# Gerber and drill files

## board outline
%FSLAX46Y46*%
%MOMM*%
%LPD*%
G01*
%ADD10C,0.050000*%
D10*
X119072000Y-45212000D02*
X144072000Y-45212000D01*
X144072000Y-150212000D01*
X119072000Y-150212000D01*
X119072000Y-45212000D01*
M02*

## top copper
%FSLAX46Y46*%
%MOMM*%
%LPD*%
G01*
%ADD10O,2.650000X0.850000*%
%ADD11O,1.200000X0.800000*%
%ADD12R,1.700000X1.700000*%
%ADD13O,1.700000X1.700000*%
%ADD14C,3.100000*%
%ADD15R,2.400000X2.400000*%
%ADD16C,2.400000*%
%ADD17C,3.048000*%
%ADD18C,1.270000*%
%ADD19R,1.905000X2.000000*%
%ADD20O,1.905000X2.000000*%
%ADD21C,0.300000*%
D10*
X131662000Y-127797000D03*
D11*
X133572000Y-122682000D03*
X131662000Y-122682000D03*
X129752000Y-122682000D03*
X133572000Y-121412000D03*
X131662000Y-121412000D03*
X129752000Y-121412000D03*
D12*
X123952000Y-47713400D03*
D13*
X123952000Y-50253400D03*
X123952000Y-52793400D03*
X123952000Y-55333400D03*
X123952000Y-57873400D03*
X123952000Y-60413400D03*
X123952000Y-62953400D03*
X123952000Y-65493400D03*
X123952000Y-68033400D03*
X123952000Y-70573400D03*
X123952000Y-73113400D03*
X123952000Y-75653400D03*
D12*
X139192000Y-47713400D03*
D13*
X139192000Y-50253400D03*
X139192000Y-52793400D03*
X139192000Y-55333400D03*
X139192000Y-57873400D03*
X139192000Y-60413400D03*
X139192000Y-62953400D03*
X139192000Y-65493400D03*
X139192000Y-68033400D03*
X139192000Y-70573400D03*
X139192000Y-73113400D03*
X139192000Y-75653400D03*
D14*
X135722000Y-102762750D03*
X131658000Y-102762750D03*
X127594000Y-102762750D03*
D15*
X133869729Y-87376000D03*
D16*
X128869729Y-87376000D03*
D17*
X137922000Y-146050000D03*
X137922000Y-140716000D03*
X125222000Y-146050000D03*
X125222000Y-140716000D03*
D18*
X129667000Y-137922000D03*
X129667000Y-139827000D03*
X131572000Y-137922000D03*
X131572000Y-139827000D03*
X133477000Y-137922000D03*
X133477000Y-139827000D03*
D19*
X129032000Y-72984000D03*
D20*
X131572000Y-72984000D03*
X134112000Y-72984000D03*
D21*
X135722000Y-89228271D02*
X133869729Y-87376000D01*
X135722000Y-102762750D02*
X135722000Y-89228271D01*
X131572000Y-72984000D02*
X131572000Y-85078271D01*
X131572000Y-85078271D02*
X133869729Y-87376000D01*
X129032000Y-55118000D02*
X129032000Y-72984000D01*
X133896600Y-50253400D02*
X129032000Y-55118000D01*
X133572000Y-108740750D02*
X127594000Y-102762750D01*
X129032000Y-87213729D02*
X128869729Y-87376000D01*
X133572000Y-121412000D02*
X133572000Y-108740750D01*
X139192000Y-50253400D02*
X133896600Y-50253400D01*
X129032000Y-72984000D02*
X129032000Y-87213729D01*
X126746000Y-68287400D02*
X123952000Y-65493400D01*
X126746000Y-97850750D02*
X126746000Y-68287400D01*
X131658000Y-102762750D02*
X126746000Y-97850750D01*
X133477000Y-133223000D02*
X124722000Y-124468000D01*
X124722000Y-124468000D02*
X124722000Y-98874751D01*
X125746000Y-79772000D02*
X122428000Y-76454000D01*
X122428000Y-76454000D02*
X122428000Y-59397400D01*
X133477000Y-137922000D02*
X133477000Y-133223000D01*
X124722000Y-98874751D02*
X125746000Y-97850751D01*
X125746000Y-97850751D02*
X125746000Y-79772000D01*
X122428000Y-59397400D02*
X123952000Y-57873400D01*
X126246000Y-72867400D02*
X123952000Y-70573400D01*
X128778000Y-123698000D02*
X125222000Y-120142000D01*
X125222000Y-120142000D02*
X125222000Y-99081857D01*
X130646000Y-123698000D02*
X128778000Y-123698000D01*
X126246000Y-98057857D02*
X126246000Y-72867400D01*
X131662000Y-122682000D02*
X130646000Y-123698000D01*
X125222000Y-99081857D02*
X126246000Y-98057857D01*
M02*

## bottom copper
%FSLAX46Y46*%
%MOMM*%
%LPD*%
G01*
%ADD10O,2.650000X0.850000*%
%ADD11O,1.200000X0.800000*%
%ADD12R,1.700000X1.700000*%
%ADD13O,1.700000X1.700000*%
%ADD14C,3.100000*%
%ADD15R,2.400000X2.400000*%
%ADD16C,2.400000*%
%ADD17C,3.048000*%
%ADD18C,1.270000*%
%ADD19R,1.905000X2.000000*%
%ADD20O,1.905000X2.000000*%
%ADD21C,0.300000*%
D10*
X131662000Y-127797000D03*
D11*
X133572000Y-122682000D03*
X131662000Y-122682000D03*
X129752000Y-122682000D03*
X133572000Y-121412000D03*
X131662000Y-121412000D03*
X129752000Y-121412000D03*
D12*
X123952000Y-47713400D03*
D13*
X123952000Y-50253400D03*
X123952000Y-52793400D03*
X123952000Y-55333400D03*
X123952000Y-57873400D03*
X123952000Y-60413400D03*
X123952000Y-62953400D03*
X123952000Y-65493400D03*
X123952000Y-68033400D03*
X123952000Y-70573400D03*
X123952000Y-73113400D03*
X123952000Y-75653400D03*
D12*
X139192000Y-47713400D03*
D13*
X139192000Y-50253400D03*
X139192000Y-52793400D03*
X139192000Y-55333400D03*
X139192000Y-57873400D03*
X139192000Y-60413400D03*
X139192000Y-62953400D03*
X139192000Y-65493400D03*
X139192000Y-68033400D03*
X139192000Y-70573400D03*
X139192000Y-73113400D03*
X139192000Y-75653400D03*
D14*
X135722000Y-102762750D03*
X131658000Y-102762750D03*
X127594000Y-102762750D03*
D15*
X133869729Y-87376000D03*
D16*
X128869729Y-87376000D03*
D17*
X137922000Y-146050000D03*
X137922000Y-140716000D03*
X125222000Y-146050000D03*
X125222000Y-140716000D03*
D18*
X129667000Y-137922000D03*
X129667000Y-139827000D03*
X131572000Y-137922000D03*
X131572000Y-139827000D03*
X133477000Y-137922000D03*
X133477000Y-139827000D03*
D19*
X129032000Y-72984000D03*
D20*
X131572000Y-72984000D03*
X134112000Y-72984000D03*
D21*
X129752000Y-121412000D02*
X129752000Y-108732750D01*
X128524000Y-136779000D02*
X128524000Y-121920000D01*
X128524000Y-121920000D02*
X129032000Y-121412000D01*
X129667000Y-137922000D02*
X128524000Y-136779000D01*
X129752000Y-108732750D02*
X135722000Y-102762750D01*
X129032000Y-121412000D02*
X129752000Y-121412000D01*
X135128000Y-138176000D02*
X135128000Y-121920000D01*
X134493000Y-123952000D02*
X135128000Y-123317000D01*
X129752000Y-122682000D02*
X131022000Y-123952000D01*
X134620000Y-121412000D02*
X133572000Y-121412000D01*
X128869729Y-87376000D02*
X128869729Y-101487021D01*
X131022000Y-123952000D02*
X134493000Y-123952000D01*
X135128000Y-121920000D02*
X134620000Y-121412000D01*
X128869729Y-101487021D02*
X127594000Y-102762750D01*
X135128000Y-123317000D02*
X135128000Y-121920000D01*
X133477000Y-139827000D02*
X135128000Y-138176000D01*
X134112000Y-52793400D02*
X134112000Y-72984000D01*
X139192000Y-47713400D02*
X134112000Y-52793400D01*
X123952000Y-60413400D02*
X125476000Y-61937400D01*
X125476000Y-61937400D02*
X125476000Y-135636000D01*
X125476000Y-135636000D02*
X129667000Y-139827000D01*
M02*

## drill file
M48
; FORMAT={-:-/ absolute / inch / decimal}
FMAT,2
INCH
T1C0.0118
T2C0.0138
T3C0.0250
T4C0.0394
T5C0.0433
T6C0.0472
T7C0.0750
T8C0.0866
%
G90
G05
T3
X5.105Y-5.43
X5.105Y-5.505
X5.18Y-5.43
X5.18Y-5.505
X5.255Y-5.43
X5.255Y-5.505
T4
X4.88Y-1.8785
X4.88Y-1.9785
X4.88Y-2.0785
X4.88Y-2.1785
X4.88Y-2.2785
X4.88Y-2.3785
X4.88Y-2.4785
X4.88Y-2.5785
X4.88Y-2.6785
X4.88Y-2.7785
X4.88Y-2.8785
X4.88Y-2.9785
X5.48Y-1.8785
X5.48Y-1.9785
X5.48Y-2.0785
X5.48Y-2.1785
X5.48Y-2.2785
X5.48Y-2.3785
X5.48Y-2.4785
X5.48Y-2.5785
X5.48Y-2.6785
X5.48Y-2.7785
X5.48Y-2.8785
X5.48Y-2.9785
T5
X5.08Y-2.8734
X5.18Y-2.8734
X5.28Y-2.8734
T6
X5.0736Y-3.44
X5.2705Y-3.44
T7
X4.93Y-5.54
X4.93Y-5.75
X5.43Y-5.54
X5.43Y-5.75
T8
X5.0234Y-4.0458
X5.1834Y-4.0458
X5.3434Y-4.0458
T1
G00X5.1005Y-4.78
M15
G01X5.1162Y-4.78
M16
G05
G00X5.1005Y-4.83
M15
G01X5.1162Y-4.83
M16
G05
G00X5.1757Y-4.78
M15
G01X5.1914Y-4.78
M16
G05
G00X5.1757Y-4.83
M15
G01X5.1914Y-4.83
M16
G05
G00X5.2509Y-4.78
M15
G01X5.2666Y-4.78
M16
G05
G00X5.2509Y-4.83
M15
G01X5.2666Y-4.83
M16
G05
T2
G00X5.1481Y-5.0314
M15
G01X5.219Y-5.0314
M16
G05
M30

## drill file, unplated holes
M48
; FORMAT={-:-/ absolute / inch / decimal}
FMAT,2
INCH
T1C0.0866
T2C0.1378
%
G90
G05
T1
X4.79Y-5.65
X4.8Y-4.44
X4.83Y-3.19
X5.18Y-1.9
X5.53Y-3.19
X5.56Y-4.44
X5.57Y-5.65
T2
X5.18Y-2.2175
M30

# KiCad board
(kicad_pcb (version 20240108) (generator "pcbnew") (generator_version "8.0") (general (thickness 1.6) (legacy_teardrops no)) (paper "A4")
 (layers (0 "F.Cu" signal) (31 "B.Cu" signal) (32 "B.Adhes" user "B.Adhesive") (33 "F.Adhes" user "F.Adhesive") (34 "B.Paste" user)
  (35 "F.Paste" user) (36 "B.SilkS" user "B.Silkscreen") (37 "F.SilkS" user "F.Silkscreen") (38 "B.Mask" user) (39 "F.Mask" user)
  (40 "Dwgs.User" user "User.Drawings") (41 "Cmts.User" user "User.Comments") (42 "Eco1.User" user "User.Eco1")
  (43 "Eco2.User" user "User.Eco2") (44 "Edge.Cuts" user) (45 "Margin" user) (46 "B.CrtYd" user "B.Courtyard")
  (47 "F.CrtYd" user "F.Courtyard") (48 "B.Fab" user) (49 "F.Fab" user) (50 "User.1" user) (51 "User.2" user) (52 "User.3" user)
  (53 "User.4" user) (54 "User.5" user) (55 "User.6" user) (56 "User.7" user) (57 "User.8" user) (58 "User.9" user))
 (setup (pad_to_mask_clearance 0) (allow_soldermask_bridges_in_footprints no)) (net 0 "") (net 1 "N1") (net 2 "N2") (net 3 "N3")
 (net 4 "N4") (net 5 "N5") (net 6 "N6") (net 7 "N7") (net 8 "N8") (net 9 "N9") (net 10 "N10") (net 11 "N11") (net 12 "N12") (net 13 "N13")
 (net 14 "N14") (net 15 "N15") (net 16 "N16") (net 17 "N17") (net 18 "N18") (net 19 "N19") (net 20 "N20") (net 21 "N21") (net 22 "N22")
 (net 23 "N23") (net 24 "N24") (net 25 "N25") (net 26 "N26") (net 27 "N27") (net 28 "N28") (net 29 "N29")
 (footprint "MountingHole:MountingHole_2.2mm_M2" (layer "F.Cu") (at 121.92 112.776)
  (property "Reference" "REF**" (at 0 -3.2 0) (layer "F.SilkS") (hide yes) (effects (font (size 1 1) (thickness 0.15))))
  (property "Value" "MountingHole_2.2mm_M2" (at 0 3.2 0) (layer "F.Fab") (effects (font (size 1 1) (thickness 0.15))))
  (pad "" np_thru_hole circle (at 0 0) (size 2.2 2.2) (drill 2.2) (layers "*.Cu" "*.Mask")))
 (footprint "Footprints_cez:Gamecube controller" (layer "F.Cu") (at 131.54 115.3668)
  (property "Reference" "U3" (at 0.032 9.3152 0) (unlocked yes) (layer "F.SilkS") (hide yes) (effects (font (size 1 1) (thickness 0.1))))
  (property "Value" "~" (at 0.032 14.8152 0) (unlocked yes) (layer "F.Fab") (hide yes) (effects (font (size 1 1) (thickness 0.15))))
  (pad "" thru_hole oval (at 0.122 12.4302) (size 2.65 0.85) (drill oval 2.15 0.35) (layers "*.Cu" "*.Mask") (remove_unused_layers no))
  (pad "1" thru_hole oval (at 2.032 7.3152) (size 1.2 0.8) (drill oval 0.7 0.3) (layers "*.Cu" "*.Mask") (remove_unused_layers no)
   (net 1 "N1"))
  (pad "2" thru_hole oval (at 0.122 7.3152) (size 1.2 0.8) (drill oval 0.7 0.3) (layers "*.Cu" "*.Mask") (remove_unused_layers no)
   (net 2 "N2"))
  (pad "3" thru_hole oval (at -1.788 7.3152) (size 1.2 0.8) (drill oval 0.7 0.3) (layers "*.Cu" "*.Mask") (remove_unused_layers no)
   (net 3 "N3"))
  (pad "4" thru_hole oval (at 2.032 6.0452) (size 1.2 0.8) (drill oval 0.7 0.3) (layers "*.Cu" "*.Mask") (remove_unused_layers no)
   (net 3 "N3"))
  (pad "5" thru_hole oval (at 0.122 6.0452) (size 1.2 0.8) (drill oval 0.7 0.3) (layers "*.Cu" "*.Mask") (remove_unused_layers no)
   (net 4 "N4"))
  (pad "6" thru_hole oval (at -1.788 6.0452) (size 1.2 0.8) (drill oval 0.7 0.3) (layers "*.Cu" "*.Mask") (remove_unused_layers no)
   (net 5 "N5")))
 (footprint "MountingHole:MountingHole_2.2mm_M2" (layer "F.Cu") (at 140.462 81.026)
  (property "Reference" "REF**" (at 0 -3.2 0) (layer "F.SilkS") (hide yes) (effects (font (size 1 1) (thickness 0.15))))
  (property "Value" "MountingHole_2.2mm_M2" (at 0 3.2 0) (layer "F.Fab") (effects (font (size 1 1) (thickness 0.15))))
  (pad "" np_thru_hole circle (at 0 0) (size 2.2 2.2) (drill 2.2) (layers "*.Cu" "*.Mask")))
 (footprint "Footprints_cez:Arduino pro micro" (layer "F.Cu") (at 129.7432 35.623)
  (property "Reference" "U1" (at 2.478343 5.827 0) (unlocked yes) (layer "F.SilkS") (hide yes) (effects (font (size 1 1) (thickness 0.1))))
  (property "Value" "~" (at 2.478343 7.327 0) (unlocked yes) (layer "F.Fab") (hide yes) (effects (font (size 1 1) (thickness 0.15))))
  (pad "1" thru_hole rect (at -5.7912 12.0904) (size 1.7 1.7) (drill 1) (layers "*.Cu" "*.Mask") (remove_unused_layers no) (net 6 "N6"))
  (pad "2" thru_hole oval (at -5.7912 14.6304) (size 1.7 1.7) (drill 1) (layers "*.Cu" "*.Mask") (remove_unused_layers no) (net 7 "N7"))
  (pad "3" thru_hole oval (at -5.7912 17.1704) (size 1.7 1.7) (drill 1) (layers "*.Cu" "*.Mask") (remove_unused_layers no) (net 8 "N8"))
  (pad "4" thru_hole oval (at -5.7912 19.7104) (size 1.7 1.7) (drill 1) (layers "*.Cu" "*.Mask") (remove_unused_layers no) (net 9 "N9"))
  (pad "5" thru_hole oval (at -5.7912 22.2504) (size 1.7 1.7) (drill 1) (layers "*.Cu" "*.Mask") (remove_unused_layers no) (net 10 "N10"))
  (pad "6" thru_hole oval (at -5.7912 24.7904) (size 1.7 1.7) (drill 1) (layers "*.Cu" "*.Mask") (remove_unused_layers no) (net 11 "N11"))
  (pad "7" thru_hole oval (at -5.7912 27.3304) (size 1.7 1.7) (drill 1) (layers "*.Cu" "*.Mask") (remove_unused_layers no) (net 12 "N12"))
  (pad "8" thru_hole oval (at -5.7912 29.8704) (size 1.7 1.7) (drill 1) (layers "*.Cu" "*.Mask") (remove_unused_layers no) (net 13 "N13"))
  (pad "9" thru_hole oval (at -5.7912 32.4104) (size 1.7 1.7) (drill 1) (layers "*.Cu" "*.Mask") (remove_unused_layers no) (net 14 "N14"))
  (pad "10" thru_hole oval (at -5.7912 34.9504) (size 1.7 1.7) (drill 1) (layers "*.Cu" "*.Mask") (remove_unused_layers no) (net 2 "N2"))
  (pad "11" thru_hole oval (at -5.7912 37.4904) (size 1.7 1.7) (drill 1) (layers "*.Cu" "*.Mask") (remove_unused_layers no) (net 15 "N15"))
  (pad "12" thru_hole oval (at -5.7912 40.0304) (size 1.7 1.7) (drill 1) (layers "*.Cu" "*.Mask") (remove_unused_layers no) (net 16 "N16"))
  (pad "13" thru_hole rect (at 9.4488 12.0904) (size 1.7 1.7) (drill 1) (layers "*.Cu" "*.Mask") (remove_unused_layers no) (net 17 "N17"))
  (pad "14" thru_hole oval (at 9.4488 14.6304) (size 1.7 1.7) (drill 1) (layers "*.Cu" "*.Mask") (remove_unused_layers no) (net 3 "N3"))
  (pad "15" thru_hole oval (at 9.4488 17.1704) (size 1.7 1.7) (drill 1) (layers "*.Cu" "*.Mask") (remove_unused_layers no) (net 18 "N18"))
  (pad "16" thru_hole oval (at 9.4488 19.7104) (size 1.7 1.7) (drill 1) (layers "*.Cu" "*.Mask") (remove_unused_layers no) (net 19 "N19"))
  (pad "17" thru_hole oval (at 9.4488 22.2504) (size 1.7 1.7) (drill 1) (layers "*.Cu" "*.Mask") (remove_unused_layers no) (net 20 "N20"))
  (pad "18" thru_hole oval (at 9.4488 24.7904) (size 1.7 1.7) (drill 1) (layers "*.Cu" "*.Mask") (remove_unused_layers no) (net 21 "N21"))
  (pad "19" thru_hole oval (at 9.4488 27.3304) (size 1.7 1.7) (drill 1) (layers "*.Cu" "*.Mask") (remove_unused_layers no) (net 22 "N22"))
  (pad "20" thru_hole oval (at 9.4488 29.8704) (size 1.7 1.7) (drill 1) (layers "*.Cu" "*.Mask") (remove_unused_layers no) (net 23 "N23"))
  (pad "21" thru_hole oval (at 9.4488 32.4104) (size 1.7 1.7) (drill 1) (layers "*.Cu" "*.Mask") (remove_unused_layers no) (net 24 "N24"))
  (pad "22" thru_hole oval (at 9.4488 34.9504) (size 1.7 1.7) (drill 1) (layers "*.Cu" "*.Mask") (remove_unused_layers no) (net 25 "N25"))
  (pad "23" thru_hole oval (at 9.4488 37.4904) (size 1.7 1.7) (drill 1) (layers "*.Cu" "*.Mask") (remove_unused_layers no) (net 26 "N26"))
  (pad "24" thru_hole oval (at 9.4488 40.0304) (size 1.7 1.7) (drill 1) (layers "*.Cu" "*.Mask") (remove_unused_layers no) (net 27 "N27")))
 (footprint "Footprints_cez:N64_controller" (layer "F.Cu") (at 131.722 118.19875 180)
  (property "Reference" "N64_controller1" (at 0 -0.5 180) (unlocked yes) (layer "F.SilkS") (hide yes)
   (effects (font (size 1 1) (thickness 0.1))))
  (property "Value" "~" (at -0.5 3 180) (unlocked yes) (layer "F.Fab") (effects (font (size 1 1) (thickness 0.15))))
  (pad "1" thru_hole circle (at -4 15.436 180) (size 3.1 3.1) (drill 2.2) (layers "*.Cu" "*.Mask") (remove_unused_layers no) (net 5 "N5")
   (solder_mask_margin 0.1016) (thermal_bridge_angle 0))
  (pad "2" thru_hole circle (at 0.064 15.436 180) (size 3.1 3.1) (drill 2.2) (layers "*.Cu" "*.Mask") (remove_unused_layers no)
   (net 13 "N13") (solder_mask_margin 0.1016) (thermal_bridge_angle 0))
  (pad "3" thru_hole circle (at 4.128 15.436 180) (size 3.1 3.1) (drill 2.2) (layers "*.Cu" "*.Mask") (remove_unused_layers no) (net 3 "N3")
   (solder_mask_margin 0.1016) (thermal_bridge_angle 0)))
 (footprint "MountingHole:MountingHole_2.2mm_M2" (layer "F.Cu") (at 131.572 48.26)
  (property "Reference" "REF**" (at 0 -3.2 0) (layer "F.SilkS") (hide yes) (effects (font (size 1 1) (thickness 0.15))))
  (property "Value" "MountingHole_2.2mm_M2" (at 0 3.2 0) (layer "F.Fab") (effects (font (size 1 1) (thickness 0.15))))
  (pad "" np_thru_hole circle (at 0 0) (size 2.2 2.2) (drill 2.2) (layers "*.Cu" "*.Mask")))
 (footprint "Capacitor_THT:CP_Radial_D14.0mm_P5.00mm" (layer "F.Cu") (at 133.869729 87.376 180)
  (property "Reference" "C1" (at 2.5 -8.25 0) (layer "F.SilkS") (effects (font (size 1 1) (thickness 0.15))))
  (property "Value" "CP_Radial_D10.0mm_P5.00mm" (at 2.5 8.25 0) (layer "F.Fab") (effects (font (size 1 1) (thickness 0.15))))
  (pad "1" thru_hole rect (at 0 0 180) (size 2.4 2.4) (drill 1.2) (layers "*.Cu" "*.Mask") (remove_unused_layers no) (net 5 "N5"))
  (pad "2" thru_hole circle (at 5 0 180) (size 2.4 2.4) (drill 1.2) (layers "*.Cu" "*.Mask") (remove_unused_layers no) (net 3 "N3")))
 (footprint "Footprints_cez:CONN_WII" (layer "F.Cu") (at 131.572 143.51 180)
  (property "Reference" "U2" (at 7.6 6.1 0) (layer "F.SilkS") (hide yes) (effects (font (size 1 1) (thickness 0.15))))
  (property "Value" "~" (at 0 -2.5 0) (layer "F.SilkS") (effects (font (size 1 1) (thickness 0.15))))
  (pad "" thru_hole circle (at -6.35 -2.54 180) (size 3.048 3.048) (drill 1.905) (layers "*.Cu" "*.Mask") (remove_unused_layers no))
  (pad "" thru_hole circle (at -6.35 2.794 180) (size 3.048 3.048) (drill 1.905) (layers "*.Cu" "*.Mask") (remove_unused_layers no))
  (pad "" thru_hole circle (at 6.35 -2.54 180) (size 3.048 3.048) (drill 1.905) (layers "*.Cu" "*.Mask") (remove_unused_layers no))
  (pad "" thru_hole circle (at 6.35 2.794 180) (size 3.048 3.048) (drill 1.905) (layers "*.Cu" "*.Mask") (remove_unused_layers no))
  (pad "1" thru_hole circle (at 1.905 5.588 180) (size 1.27 1.27) (drill 0.635) (layers "*.Cu" "*.Mask") (remove_unused_layers no)
   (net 5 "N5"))
  (pad "2" thru_hole circle (at 1.905 3.683 180) (size 1.27 1.27) (drill 0.635) (layers "*.Cu" "*.Mask") (remove_unused_layers no)
   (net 11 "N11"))
  (pad "3" thru_hole circle (at 0 5.588 180) (size 1.27 1.27) (drill 0.635) (layers "*.Cu" "*.Mask") (remove_unused_layers no)
   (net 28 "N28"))
  (pad "4" thru_hole circle (at 0 3.683 180) (size 1.27 1.27) (drill 0.635) (layers "*.Cu" "*.Mask") (remove_unused_layers no)
   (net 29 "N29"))
  (pad "5" thru_hole circle (at -1.905 5.588 180) (size 1.27 1.27) (drill 0.635) (layers "*.Cu" "*.Mask") (remove_unused_layers no)
   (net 10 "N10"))
  (pad "6" thru_hole circle (at -1.905 3.683 180) (size 1.27 1.27) (drill 0.635) (layers "*.Cu" "*.Mask") (remove_unused_layers no)
   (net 3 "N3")))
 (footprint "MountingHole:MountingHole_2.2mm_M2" (layer "F.Cu") (at 141.224 112.776)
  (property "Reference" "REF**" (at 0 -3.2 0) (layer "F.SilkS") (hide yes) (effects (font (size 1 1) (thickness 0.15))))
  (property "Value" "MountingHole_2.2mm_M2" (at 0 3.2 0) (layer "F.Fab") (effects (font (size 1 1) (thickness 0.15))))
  (pad "" np_thru_hole circle (at 0 0) (size 2.2 2.2) (drill 2.2) (layers "*.Cu" "*.Mask")))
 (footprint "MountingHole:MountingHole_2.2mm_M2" (layer "F.Cu") (at 121.666 143.51)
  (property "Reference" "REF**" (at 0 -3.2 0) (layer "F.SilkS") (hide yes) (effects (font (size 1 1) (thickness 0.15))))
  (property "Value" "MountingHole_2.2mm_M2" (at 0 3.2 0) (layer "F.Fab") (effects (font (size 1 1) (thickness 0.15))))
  (pad "" np_thru_hole circle (at 0 0) (size 2.2 2.2) (drill 2.2) (layers "*.Cu" "*.Mask")))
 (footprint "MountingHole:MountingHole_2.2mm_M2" (layer "F.Cu") (at 141.478 143.51)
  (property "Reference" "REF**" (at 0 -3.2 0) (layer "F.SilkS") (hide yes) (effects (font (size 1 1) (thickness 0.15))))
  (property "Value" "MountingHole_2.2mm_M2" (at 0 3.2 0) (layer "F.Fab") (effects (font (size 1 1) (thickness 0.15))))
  (pad "" np_thru_hole circle (at 0 0) (size 2.2 2.2) (drill 2.2) (layers "*.Cu" "*.Mask")))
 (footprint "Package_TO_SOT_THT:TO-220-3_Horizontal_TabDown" (layer "F.Cu") (at 129.032 72.984)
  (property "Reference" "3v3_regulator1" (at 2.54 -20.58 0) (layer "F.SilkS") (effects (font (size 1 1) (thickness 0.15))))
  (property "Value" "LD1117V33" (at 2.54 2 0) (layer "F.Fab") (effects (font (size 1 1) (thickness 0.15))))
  (pad "" np_thru_hole oval (at 2.54 -16.66) (size 3.5 3.5) (drill 3.5) (layers "*.Cu" "*.Mask"))
  (pad "1" thru_hole rect (at 0 0) (size 1.905 2) (drill 1.1) (layers "*.Cu" "*.Mask") (remove_unused_layers no) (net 3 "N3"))
  (pad "2" thru_hole oval (at 2.54 0) (size 1.905 2) (drill 1.1) (layers "*.Cu" "*.Mask") (remove_unused_layers no) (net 5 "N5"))
  (pad "3" thru_hole oval (at 5.08 0) (size 1.905 2) (drill 1.1) (layers "*.Cu" "*.Mask") (remove_unused_layers no) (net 17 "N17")))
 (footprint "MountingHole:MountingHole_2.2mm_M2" (layer "F.Cu") (at 122.682 81.026)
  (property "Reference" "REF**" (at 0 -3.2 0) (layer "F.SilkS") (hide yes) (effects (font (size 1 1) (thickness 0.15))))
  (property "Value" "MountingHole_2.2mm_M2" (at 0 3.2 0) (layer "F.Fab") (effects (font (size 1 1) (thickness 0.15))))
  (pad "" np_thru_hole circle (at 0 0) (size 2.2 2.2) (drill 2.2) (layers "F&B.Cu" "*.Mask")))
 (gr_rect (start 119.072 45.212) (end 144.072 150.212) (stroke (width 0.05) (type default)) (fill none) (layer "Edge.Cuts"))
 (segment (start 135.722 89.228271) (end 133.869729 87.376) (width 0.3) (layer "F.Cu") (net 5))
 (segment (start 135.722 102.76275) (end 135.722 89.228271) (width 0.3) (layer "F.Cu") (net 5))
 (segment (start 131.572 72.984) (end 131.572 85.078271) (width 0.3) (layer "F.Cu") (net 5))
 (segment (start 131.572 85.078271) (end 133.869729 87.376) (width 0.3) (layer "F.Cu") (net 5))
 (segment (start 129.752 121.412) (end 129.752 108.73275) (width 0.3) (layer "B.Cu") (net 5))
 (segment (start 128.524 136.779) (end 128.524 121.92) (width 0.3) (layer "B.Cu") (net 5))
 (segment (start 128.524 121.92) (end 129.032 121.412) (width 0.3) (layer "B.Cu") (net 5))
 (segment (start 129.667 137.922) (end 128.524 136.779) (width 0.3) (layer "B.Cu") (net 5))
 (segment (start 129.752 108.73275) (end 135.722 102.76275) (width 0.3) (layer "B.Cu") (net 5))
 (segment (start 129.032 121.412) (end 129.752 121.412) (width 0.3) (layer "B.Cu") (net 5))
 (segment (start 129.032 55.118) (end 129.032 72.984) (width 0.3) (layer "F.Cu") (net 3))
 (segment (start 133.8966 50.2534) (end 129.032 55.118) (width 0.3) (layer "F.Cu") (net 3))
 (segment (start 133.572 108.74075) (end 127.594 102.76275) (width 0.3) (layer "F.Cu") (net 3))
 (segment (start 129.032 87.213729) (end 128.869729 87.376) (width 0.3) (layer "F.Cu") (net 3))
 (segment (start 133.572 121.412) (end 133.572 108.74075) (width 0.3) (layer "F.Cu") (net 3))
 (segment (start 139.192 50.2534) (end 133.8966 50.2534) (width 0.3) (layer "F.Cu") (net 3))
 (segment (start 129.032 72.984) (end 129.032 87.213729) (width 0.3) (layer "F.Cu") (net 3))
 (segment (start 135.128 138.176) (end 135.128 121.92) (width 0.3) (layer "B.Cu") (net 3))
 (segment (start 134.493 123.952) (end 135.128 123.317) (width 0.3) (layer "B.Cu") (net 3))
 (segment (start 129.752 122.682) (end 131.022 123.952) (width 0.3) (layer "B.Cu") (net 3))
 (segment (start 134.62 121.412) (end 133.572 121.412) (width 0.3) (layer "B.Cu") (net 3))
 (segment (start 128.869729 87.376) (end 128.869729 101.487021) (width 0.3) (layer "B.Cu") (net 3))
 (segment (start 131.022 123.952) (end 134.493 123.952) (width 0.3) (layer "B.Cu") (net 3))
 (segment (start 135.128 121.92) (end 134.62 121.412) (width 0.3) (layer "B.Cu") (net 3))
 (segment (start 128.869729 101.487021) (end 127.594 102.76275) (width 0.3) (layer "B.Cu") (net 3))
 (segment (start 135.128 123.317) (end 135.128 121.92) (width 0.3) (layer "B.Cu") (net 3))
 (segment (start 133.477 139.827) (end 135.128 138.176) (width 0.3) (layer "B.Cu") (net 3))
 (segment (start 134.112 52.7934) (end 134.112 72.984) (width 0.3) (layer "B.Cu") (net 17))
 (segment (start 139.192 47.7134) (end 134.112 52.7934) (width 0.3) (layer "B.Cu") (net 17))
 (segment (start 126.746 68.2874) (end 123.952 65.4934) (width 0.3) (layer "F.Cu") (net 13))
 (segment (start 126.746 97.85075) (end 126.746 68.2874) (width 0.3) (layer "F.Cu") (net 13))
 (segment (start 131.658 102.76275) (end 126.746 97.85075) (width 0.3) (layer "F.Cu") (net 13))
 (segment (start 123.952 60.4134) (end 125.476 61.9374) (width 0.3) (layer "B.Cu") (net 11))
 (segment (start 125.476 61.9374) (end 125.476 135.636) (width 0.3) (layer "B.Cu") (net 11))
 (segment (start 125.476 135.636) (end 129.667 139.827) (width 0.3) (layer "B.Cu") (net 11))
 (segment (start 133.477 133.223) (end 124.722 124.468) (width 0.3) (layer "F.Cu") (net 10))
 (segment (start 124.722 124.468) (end 124.722 98.874751) (width 0.3) (layer "F.Cu") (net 10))
 (segment (start 125.746 79.772) (end 122.428 76.454) (width 0.3) (layer "F.Cu") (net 10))
 (segment (start 122.428 76.454) (end 122.428 59.3974) (width 0.3) (layer "F.Cu") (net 10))
 (segment (start 133.477 137.922) (end 133.477 133.223) (width 0.3) (layer "F.Cu") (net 10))
 (segment (start 124.722 98.874751) (end 125.746 97.850751) (width 0.3) (layer "F.Cu") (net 10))
 (segment (start 125.746 97.850751) (end 125.746 79.772) (width 0.3) (layer "F.Cu") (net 10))
 (segment (start 122.428 59.3974) (end 123.952 57.8734) (width 0.3) (layer "F.Cu") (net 10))
 (segment (start 126.246 72.8674) (end 123.952 70.5734) (width 0.3) (layer "F.Cu") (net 2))
 (segment (start 128.778 123.698) (end 125.222 120.142) (width 0.3) (layer "F.Cu") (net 2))
 (segment (start 125.222 120.142) (end 125.222 99.081857) (width 0.3) (layer "F.Cu") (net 2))
 (segment (start 130.646 123.698) (end 128.778 123.698) (width 0.3) (layer "F.Cu") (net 2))
 (segment (start 126.246 98.057857) (end 126.246 72.8674) (width 0.3) (layer "F.Cu") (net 2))
 (segment (start 131.662 122.682) (end 130.646 123.698) (width 0.3) (layer "F.Cu") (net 2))
 (segment (start 125.222 99.081857) (end 126.246 98.057857) (width 0.3) (layer "F.Cu") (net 2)))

